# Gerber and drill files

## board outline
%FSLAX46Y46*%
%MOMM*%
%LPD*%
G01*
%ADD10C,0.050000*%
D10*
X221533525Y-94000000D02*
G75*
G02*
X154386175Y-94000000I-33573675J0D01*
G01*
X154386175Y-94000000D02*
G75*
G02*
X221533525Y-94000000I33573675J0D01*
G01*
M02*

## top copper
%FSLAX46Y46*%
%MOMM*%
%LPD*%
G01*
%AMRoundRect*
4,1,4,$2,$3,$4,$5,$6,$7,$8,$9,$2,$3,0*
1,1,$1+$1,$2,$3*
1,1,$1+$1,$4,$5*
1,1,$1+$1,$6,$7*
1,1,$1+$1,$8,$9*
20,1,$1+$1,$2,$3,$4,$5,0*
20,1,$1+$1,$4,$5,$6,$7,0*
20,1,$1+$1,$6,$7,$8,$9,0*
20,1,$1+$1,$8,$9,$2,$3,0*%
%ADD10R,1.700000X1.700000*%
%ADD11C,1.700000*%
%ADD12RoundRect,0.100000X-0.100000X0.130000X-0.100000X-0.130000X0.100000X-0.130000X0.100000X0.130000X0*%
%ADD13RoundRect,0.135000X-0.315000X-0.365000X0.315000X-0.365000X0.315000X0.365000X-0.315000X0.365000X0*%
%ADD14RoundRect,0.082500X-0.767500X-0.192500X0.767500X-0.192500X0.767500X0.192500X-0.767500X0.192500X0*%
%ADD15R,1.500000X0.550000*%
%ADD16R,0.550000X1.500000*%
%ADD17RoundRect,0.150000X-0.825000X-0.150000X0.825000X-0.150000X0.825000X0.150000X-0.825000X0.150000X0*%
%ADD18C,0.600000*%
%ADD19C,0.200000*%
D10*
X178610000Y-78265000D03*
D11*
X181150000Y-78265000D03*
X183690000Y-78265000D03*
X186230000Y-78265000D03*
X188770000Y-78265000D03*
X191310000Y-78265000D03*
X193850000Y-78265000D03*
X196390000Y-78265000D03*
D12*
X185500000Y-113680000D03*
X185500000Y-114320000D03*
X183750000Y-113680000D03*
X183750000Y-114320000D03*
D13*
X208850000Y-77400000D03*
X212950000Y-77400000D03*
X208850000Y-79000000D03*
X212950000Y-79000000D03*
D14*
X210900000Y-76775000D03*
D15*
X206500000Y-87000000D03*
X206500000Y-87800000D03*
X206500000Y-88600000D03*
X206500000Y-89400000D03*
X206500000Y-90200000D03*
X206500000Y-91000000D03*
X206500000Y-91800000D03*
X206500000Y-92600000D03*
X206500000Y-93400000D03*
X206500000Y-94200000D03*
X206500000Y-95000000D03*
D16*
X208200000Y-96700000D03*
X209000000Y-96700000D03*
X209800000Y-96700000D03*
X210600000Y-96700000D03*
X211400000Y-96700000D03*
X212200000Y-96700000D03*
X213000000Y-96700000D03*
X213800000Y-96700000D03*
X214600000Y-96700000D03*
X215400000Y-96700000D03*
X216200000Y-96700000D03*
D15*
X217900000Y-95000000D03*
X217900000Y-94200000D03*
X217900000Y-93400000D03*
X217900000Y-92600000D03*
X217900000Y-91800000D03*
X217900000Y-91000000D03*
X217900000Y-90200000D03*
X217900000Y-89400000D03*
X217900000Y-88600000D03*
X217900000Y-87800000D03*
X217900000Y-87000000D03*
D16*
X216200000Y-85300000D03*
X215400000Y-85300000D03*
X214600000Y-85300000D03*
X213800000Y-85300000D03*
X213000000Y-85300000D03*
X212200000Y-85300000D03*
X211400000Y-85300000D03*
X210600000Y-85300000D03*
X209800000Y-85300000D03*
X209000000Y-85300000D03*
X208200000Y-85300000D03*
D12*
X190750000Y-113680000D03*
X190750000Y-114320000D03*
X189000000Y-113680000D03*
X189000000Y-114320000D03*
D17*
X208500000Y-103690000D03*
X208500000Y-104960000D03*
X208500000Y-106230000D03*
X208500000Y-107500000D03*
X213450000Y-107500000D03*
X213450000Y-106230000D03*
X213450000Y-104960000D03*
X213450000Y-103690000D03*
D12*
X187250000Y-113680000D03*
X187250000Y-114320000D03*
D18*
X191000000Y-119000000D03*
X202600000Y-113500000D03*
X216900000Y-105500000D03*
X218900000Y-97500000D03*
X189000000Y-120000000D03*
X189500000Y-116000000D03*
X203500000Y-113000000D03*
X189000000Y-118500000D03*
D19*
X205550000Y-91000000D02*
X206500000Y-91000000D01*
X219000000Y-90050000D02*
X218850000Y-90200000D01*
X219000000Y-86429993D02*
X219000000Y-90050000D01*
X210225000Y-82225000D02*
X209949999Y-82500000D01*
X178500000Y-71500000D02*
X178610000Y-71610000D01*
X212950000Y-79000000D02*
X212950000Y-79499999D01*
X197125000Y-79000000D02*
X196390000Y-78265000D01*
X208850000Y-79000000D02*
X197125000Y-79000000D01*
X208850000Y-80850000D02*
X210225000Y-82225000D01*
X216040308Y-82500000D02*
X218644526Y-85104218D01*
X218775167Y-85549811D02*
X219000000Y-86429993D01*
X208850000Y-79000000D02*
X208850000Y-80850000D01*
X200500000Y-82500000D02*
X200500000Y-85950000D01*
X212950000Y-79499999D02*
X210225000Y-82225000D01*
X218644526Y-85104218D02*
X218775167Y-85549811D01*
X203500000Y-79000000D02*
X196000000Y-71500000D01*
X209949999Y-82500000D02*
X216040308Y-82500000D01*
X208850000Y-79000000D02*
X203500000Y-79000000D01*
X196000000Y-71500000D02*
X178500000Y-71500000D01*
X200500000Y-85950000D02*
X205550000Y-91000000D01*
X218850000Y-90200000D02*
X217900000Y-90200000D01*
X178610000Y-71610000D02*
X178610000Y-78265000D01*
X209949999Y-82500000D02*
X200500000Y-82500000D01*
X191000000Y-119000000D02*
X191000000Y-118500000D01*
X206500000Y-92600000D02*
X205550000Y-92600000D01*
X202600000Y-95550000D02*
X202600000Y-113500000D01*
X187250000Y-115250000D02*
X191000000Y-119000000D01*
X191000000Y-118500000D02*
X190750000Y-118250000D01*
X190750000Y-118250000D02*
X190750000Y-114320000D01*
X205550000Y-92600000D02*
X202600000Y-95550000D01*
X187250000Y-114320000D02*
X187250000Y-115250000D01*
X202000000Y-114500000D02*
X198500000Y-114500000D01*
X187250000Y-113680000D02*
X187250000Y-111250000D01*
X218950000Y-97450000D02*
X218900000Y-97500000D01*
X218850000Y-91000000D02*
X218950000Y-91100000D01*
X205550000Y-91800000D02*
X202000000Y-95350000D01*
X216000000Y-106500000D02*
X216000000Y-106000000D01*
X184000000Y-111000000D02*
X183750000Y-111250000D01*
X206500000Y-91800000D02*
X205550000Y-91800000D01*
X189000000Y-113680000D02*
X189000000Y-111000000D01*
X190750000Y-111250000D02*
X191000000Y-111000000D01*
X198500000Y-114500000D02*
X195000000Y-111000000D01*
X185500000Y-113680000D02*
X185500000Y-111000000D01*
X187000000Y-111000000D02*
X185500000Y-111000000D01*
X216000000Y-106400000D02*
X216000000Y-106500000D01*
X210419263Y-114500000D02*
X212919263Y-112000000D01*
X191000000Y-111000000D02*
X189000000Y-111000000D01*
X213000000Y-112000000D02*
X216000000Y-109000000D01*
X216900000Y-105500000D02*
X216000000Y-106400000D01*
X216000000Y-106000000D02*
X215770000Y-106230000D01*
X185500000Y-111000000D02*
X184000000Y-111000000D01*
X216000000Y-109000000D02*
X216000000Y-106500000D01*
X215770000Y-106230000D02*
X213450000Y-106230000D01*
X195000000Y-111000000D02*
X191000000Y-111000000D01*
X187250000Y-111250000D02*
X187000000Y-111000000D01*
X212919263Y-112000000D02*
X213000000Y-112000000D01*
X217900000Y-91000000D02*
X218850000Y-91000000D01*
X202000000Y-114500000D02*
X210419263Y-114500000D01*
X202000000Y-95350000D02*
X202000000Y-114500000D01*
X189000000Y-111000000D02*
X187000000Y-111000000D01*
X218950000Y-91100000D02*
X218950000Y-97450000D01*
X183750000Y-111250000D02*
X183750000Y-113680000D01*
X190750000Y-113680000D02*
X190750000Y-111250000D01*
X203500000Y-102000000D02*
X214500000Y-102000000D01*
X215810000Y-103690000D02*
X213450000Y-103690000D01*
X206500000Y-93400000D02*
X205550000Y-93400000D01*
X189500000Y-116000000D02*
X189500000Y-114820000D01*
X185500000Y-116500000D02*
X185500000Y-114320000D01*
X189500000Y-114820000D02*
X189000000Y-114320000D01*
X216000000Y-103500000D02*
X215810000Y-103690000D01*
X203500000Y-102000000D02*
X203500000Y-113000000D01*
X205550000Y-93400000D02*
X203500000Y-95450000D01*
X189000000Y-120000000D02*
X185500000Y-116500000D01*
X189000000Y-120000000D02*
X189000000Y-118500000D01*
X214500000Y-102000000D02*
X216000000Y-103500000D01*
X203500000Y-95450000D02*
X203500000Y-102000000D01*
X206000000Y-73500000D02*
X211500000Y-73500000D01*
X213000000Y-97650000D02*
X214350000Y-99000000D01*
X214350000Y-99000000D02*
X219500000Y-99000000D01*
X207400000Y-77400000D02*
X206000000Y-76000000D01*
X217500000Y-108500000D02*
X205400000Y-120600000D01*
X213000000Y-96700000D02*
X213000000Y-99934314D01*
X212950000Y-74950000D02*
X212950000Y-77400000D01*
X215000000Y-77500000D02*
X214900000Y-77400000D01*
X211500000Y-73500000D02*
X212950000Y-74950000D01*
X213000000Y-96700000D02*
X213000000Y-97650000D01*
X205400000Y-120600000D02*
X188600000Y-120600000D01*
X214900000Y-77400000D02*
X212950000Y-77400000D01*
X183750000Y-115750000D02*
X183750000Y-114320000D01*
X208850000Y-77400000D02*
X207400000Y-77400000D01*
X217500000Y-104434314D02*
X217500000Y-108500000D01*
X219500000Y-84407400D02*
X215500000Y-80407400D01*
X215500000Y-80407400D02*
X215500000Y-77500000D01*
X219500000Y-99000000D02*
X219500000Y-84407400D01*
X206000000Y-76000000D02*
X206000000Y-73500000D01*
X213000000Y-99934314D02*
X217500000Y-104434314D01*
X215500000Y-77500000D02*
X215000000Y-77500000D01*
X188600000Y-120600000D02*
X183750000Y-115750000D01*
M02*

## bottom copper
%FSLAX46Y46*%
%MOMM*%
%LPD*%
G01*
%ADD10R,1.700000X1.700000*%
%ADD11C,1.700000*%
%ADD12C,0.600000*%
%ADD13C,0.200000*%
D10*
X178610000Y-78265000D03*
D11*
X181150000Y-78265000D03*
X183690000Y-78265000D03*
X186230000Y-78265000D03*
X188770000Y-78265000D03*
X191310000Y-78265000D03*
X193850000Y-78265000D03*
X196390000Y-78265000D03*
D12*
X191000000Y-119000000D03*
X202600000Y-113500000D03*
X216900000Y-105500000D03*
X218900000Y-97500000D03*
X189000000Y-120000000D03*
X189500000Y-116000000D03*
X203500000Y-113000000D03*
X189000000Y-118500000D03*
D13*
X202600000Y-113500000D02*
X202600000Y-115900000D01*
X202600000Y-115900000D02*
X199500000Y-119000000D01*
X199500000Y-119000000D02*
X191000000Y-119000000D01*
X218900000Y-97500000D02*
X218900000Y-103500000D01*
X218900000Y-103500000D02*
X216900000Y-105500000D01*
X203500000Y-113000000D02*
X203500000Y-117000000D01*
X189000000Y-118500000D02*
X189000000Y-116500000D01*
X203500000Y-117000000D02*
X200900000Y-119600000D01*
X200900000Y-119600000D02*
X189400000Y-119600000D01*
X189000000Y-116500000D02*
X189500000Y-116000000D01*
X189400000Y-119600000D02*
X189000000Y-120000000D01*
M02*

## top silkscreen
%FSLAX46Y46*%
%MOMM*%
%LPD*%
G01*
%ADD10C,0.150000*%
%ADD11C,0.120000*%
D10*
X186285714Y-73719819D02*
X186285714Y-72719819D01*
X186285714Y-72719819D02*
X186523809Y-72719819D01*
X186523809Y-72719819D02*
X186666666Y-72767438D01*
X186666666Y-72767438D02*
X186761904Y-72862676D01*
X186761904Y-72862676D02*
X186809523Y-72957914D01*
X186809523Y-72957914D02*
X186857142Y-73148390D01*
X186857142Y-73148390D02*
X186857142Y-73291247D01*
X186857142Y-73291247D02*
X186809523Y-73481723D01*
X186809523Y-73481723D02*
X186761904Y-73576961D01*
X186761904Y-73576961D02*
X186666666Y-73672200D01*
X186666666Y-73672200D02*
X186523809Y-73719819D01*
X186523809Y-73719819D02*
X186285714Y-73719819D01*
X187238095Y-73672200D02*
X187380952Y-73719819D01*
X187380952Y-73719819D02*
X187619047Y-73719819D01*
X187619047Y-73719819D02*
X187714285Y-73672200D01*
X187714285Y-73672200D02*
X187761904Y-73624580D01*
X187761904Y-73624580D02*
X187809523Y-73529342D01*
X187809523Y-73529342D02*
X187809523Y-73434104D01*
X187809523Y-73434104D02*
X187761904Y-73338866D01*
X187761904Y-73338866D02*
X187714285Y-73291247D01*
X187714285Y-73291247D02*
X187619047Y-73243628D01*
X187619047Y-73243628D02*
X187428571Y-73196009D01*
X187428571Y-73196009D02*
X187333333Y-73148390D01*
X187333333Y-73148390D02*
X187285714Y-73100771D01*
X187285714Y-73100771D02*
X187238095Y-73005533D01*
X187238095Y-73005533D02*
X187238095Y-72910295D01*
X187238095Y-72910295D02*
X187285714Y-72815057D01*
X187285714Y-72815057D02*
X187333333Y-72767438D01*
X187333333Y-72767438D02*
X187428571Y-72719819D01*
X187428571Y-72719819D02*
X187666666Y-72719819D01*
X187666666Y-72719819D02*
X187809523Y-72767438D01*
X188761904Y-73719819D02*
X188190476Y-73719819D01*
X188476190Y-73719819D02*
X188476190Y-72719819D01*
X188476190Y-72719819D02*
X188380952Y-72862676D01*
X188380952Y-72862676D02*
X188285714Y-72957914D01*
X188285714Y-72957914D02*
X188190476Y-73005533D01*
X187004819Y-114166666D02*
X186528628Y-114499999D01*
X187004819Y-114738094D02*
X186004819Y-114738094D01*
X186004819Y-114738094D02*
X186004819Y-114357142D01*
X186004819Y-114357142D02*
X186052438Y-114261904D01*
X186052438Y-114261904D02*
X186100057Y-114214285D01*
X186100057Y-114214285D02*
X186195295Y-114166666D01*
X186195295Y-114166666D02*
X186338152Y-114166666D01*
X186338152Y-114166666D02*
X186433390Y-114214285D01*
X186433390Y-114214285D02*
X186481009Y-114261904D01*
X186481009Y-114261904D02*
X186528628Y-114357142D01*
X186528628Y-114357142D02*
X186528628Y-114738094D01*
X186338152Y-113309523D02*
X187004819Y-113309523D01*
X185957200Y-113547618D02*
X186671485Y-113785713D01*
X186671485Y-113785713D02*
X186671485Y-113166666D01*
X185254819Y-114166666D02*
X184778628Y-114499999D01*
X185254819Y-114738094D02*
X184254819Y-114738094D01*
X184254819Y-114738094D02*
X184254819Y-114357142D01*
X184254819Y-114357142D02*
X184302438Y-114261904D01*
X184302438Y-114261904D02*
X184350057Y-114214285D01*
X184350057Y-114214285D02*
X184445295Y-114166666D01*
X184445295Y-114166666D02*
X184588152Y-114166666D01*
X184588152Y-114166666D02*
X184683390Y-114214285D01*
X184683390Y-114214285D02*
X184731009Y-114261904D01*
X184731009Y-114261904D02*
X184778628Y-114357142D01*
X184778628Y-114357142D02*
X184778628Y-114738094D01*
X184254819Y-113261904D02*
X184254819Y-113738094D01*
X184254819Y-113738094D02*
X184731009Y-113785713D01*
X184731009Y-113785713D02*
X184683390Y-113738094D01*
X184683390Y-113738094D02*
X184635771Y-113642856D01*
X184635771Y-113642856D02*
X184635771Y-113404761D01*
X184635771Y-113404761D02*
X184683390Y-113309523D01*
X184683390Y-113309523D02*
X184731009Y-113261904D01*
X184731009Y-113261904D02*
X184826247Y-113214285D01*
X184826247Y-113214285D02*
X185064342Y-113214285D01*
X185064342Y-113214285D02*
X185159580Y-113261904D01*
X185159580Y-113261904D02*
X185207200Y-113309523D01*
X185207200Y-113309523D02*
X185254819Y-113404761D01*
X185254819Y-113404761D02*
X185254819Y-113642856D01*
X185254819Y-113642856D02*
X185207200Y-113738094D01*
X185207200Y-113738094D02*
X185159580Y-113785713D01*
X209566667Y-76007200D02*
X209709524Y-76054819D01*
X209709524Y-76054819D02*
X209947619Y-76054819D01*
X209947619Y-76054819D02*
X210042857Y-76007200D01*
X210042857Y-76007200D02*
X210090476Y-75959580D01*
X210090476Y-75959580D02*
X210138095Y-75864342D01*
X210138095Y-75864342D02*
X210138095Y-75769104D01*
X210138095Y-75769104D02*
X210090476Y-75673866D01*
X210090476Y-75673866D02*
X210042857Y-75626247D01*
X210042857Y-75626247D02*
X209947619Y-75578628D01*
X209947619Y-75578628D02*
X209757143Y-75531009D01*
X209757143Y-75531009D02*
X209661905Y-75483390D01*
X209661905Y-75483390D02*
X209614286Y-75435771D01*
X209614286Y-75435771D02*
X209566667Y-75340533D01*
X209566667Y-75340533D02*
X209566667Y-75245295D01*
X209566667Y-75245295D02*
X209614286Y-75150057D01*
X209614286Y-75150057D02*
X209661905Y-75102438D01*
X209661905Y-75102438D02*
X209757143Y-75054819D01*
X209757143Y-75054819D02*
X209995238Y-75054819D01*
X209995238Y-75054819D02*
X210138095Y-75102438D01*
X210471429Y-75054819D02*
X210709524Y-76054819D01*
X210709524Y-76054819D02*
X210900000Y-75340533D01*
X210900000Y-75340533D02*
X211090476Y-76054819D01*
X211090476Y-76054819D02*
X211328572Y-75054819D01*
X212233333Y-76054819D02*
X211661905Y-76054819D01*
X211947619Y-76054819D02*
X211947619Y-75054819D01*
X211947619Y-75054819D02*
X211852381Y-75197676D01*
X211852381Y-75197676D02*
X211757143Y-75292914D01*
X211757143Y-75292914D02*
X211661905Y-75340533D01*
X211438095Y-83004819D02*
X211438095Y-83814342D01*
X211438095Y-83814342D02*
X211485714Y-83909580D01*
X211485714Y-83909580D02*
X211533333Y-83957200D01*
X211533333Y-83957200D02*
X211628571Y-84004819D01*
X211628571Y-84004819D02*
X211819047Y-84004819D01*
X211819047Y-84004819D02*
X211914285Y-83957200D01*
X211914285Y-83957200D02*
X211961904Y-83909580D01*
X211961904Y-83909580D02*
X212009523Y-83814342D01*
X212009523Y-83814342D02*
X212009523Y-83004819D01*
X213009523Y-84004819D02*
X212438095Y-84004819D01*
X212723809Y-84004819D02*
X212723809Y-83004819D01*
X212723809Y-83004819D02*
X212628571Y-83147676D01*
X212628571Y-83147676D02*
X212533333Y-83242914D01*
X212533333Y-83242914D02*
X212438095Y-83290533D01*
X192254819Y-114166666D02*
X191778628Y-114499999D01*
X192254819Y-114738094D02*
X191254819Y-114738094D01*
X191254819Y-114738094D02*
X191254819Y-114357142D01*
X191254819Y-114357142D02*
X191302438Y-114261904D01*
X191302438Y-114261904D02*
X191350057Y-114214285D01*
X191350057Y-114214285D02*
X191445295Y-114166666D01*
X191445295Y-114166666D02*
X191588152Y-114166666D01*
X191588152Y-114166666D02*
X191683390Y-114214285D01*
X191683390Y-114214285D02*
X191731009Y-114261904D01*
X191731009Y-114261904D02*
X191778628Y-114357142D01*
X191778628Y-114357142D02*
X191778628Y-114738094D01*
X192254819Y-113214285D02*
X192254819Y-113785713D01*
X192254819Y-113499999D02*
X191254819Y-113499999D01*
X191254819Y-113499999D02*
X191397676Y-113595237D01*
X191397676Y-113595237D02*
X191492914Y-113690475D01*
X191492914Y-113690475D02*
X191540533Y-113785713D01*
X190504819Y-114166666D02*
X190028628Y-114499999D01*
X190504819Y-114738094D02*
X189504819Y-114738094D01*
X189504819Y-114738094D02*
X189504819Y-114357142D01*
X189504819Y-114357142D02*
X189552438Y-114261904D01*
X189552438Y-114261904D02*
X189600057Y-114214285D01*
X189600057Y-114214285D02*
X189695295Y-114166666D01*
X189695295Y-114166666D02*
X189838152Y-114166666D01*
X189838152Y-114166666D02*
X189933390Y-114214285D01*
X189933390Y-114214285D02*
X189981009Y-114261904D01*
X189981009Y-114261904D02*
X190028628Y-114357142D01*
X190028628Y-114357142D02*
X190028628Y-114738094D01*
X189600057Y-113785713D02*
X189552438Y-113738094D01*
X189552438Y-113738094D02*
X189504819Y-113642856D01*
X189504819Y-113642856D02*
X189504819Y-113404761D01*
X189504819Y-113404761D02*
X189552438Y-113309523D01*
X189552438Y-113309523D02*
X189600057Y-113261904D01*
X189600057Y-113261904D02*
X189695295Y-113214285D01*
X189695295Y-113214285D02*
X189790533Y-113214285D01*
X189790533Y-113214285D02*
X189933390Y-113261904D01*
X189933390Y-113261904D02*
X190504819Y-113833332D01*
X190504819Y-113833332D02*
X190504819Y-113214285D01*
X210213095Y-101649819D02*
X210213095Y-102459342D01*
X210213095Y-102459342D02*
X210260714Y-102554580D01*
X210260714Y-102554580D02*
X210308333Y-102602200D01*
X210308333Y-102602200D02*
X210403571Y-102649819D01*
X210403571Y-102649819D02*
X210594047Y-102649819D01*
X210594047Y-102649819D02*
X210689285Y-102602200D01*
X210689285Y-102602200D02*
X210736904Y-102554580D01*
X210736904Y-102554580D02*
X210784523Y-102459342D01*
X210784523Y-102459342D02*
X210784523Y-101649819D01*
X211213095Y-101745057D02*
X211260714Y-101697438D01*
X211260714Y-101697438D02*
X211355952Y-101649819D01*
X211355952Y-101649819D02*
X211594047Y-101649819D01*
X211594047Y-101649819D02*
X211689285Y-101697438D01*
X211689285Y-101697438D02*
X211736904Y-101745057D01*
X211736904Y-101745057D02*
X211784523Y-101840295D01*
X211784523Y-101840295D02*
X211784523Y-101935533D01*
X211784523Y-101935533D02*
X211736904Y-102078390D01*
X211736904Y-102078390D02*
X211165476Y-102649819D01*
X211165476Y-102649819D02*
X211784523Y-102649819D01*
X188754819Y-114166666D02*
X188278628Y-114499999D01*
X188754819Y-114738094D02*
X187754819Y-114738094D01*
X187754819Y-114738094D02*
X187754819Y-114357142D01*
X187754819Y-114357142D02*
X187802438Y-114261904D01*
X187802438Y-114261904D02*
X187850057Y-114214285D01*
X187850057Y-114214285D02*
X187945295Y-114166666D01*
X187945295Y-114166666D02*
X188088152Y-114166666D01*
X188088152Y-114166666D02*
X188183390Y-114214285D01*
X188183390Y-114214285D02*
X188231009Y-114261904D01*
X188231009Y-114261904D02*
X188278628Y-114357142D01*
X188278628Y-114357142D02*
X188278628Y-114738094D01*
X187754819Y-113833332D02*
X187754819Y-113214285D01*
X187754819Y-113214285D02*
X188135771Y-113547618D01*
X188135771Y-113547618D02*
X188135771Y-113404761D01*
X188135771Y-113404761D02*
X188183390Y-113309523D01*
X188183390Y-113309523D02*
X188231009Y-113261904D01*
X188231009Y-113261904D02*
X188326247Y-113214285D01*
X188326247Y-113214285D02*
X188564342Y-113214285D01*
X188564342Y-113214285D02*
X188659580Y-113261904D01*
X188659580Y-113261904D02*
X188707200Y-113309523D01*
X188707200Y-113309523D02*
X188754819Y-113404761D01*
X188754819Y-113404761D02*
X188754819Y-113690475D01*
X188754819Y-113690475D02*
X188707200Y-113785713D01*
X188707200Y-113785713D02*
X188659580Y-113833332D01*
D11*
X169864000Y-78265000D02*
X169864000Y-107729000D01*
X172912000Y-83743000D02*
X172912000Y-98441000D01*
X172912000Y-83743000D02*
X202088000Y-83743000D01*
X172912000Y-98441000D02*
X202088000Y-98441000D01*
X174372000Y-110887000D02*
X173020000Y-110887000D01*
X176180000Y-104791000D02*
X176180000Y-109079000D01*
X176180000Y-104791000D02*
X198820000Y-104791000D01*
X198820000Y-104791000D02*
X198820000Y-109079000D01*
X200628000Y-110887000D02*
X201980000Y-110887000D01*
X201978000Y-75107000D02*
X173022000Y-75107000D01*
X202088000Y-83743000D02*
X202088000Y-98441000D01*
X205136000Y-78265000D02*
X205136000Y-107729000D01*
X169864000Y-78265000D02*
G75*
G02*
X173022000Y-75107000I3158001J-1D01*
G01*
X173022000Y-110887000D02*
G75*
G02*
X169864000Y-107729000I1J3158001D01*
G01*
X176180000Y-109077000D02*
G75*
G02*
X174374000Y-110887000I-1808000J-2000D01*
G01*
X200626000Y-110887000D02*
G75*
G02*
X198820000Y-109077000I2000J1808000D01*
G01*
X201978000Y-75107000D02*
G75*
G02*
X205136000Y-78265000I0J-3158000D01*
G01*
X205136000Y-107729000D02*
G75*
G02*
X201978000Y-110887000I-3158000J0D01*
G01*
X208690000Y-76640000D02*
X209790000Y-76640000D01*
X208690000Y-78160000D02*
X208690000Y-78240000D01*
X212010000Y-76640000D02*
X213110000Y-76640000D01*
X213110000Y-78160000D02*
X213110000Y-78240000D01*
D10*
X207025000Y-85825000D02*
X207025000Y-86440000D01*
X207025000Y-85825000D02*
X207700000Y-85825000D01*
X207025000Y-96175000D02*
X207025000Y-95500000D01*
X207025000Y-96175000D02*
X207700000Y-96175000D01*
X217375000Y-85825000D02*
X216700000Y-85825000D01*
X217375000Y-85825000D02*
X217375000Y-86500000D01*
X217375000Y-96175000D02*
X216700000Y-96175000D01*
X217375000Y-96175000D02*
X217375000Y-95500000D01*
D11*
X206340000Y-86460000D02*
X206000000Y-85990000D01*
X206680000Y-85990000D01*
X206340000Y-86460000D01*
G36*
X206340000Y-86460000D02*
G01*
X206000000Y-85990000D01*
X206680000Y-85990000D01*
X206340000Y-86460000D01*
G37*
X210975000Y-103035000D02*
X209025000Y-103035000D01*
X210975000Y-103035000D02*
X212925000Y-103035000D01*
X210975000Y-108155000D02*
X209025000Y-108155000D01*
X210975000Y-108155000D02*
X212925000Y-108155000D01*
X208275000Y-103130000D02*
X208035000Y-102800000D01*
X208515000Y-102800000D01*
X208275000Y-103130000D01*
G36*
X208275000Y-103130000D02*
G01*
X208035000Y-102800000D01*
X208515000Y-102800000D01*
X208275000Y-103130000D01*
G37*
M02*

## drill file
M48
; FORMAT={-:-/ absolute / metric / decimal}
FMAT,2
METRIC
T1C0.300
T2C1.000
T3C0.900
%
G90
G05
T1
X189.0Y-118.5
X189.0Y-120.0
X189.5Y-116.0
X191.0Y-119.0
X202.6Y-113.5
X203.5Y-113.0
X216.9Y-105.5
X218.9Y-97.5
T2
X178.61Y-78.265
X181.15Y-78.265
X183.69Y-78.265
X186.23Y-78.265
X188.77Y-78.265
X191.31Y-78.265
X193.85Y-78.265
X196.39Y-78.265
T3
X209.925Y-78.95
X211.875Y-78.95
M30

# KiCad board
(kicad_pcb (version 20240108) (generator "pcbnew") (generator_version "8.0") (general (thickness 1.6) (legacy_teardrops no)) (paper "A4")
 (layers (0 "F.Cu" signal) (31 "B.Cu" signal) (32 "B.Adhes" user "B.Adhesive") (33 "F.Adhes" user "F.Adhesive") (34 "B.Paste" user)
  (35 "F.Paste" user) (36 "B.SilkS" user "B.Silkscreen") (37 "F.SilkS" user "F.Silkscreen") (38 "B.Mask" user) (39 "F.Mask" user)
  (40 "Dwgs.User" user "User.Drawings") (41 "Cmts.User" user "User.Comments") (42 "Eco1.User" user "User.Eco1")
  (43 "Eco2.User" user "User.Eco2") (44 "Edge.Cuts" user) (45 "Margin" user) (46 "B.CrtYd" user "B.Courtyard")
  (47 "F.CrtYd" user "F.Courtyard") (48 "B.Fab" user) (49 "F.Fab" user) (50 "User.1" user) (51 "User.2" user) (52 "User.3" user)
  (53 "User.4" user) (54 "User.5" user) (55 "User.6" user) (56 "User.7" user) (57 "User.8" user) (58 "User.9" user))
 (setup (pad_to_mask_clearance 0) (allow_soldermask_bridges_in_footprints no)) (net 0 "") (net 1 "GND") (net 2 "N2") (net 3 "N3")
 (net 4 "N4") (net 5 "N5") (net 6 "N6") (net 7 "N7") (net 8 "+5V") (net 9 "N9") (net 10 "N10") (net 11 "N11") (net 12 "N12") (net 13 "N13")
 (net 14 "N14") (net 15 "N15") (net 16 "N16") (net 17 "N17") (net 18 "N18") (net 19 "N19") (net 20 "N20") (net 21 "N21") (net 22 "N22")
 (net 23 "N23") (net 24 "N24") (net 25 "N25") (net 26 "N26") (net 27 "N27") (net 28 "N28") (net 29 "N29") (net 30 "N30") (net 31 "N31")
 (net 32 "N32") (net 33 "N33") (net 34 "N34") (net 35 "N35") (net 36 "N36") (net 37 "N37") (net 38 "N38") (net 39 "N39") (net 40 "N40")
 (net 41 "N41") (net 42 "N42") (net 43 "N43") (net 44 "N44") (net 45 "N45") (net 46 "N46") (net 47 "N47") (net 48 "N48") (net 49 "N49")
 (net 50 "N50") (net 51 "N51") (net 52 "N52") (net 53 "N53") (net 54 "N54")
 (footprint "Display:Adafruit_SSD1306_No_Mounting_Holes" (layer "F.Cu") (at 178.61 78.265)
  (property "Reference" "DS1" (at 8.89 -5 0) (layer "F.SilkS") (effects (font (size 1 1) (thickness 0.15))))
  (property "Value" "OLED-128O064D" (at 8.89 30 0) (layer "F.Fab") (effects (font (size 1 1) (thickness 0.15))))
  (fp_line (start -8.746 0) (end -8.746 29.464) (stroke (width 0.12) (type solid)) (layer "F.SilkS"))
  (fp_line (start -5.698 5.478) (end -5.698 20.176) (stroke (width 0.12) (type solid)) (layer "F.SilkS"))
  (fp_line (start -5.698 5.478) (end 23.478 5.478) (stroke (width 0.12) (type solid)) (layer "F.SilkS"))
  (fp_line (start -5.698 20.176) (end 23.478 20.176) (stroke (width 0.12) (type solid)) (layer "F.SilkS"))
  (fp_line (start -4.238 32.622) (end -5.59 32.622) (stroke (width 0.12) (type solid)) (layer "F.SilkS"))
  (fp_line (start -2.43 26.526) (end -2.43 30.814) (stroke (width 0.12) (type solid)) (layer "F.SilkS"))
  (fp_line (start -2.43 26.526) (end 20.21 26.526) (stroke (width 0.12) (type solid)) (layer "F.SilkS"))
  (fp_line (start 20.21 26.526) (end 20.21 30.814) (stroke (width 0.12) (type solid)) (layer "F.SilkS"))
  (fp_line (start 22.018 32.622) (end 23.37 32.622) (stroke (width 0.12) (type solid)) (layer "F.SilkS"))
  (fp_line (start 23.368 -3.158) (end -5.588 -3.158) (stroke (width 0.12) (type solid)) (layer "F.SilkS"))
  (fp_line (start 23.478 5.478) (end 23.478 20.176) (stroke (width 0.12) (type solid)) (layer "F.SilkS"))
  (fp_line (start 26.526 0) (end 26.526 29.464) (stroke (width 0.12) (type solid)) (layer "F.SilkS"))
  (fp_arc (start -8.746 0) (mid -7.821043 -2.233043) (end -5.588 -3.158) (stroke (width 0.12) (type solid)) (layer "F.SilkS"))
  (fp_arc (start -5.588 32.622) (mid -7.821043 31.697043) (end -8.746 29.464) (stroke (width 0.12) (type solid)) (layer "F.SilkS"))
  (fp_arc (start -2.43 30.812) (mid -2.958137 32.091035) (end -4.236 32.622) (stroke (width 0.12) (type solid)) (layer "F.SilkS"))
  (fp_arc (start 22.016 32.622) (mid 20.738137 32.091035) (end 20.21 30.812) (stroke (width 0.12) (type solid)) (layer "F.SilkS"))
  (fp_arc (start 23.368 -3.158) (mid 25.601043 -2.233043) (end 26.526 0) (stroke (width 0.12) (type solid)) (layer "F.SilkS"))
  (fp_arc (start 26.526 29.464) (mid 25.601043 31.697043) (end 23.368 32.622) (stroke (width 0.12) (type solid)) (layer "F.SilkS"))
  (pad "1" thru_hole rect (at 0 0) (size 1.7 1.7) (drill 1) (layers "*.Cu" "*.Mask") (remove_unused_layers no) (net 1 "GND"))
  (pad "2" thru_hole circle (at 2.54 0) (size 1.7 1.7) (drill 1) (layers "*.Cu" "*.Mask") (remove_unused_layers no) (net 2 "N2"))
  (pad "3" thru_hole circle (at 5.08 0) (size 1.7 1.7) (drill 1) (layers "*.Cu" "*.Mask") (remove_unused_layers no) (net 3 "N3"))
  (pad "4" thru_hole circle (at 7.62 0) (size 1.7 1.7) (drill 1) (layers "*.Cu" "*.Mask") (remove_unused_layers no) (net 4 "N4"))
  (pad "5" thru_hole circle (at 10.16 0) (size 1.7 1.7) (drill 1) (layers "*.Cu" "*.Mask") (remove_unused_layers no) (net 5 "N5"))
  (pad "6" thru_hole circle (at 12.7 0) (size 1.7 1.7) (drill 1) (layers "*.Cu" "*.Mask") (remove_unused_layers no) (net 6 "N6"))
  (pad "7" thru_hole circle (at 15.24 0) (size 1.7 1.7) (drill 1) (layers "*.Cu" "*.Mask") (remove_unused_layers no) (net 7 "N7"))
  (pad "8" thru_hole circle (at 17.78 0) (size 1.7 1.7) (drill 1) (layers "*.Cu" "*.Mask") (remove_unused_layers no) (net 1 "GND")))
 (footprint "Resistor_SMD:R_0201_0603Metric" (layer "F.Cu") (at 185.5 114 -90)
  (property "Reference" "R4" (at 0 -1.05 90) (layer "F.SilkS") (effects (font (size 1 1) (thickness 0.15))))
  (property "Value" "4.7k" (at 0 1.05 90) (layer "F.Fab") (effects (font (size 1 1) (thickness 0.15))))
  (pad "" smd roundrect (at -0.345 0 270) (size 0.318 0.36) (layers "F.Paste") (roundrect_rratio 0.25))
  (pad "" smd roundrect (at 0.345 0 270) (size 0.318 0.36) (layers "F.Paste") (roundrect_rratio 0.25))
  (pad "1" smd roundrect (at -0.32 0 270) (size 0.46 0.4) (layers "F.Cu" "F.Mask") (roundrect_rratio 0.25) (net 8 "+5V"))
  (pad "2" smd roundrect (at 0.32 0 270) (size 0.46 0.4) (layers "F.Cu" "F.Mask") (roundrect_rratio 0.25) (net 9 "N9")))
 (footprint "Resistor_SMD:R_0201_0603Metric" (layer "F.Cu") (at 183.75 114 -90)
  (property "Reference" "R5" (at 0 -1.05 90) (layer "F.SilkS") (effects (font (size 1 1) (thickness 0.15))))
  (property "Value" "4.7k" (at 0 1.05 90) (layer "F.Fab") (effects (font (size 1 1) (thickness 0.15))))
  (pad "" smd roundrect (at -0.345 0 270) (size 0.318 0.36) (layers "F.Paste") (roundrect_rratio 0.25))
  (pad "" smd roundrect (at 0.345 0 270) (size 0.318 0.36) (layers "F.Paste") (roundrect_rratio 0.25))
  (pad "1" smd roundrect (at -0.32 0 270) (size 0.46 0.4) (layers "F.Cu" "F.Mask") (roundrect_rratio 0.25) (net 8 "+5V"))
  (pad "2" smd roundrect (at 0.32 0 270) (size 0.46 0.4) (layers "F.Cu" "F.Mask") (roundrect_rratio 0.25) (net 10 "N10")))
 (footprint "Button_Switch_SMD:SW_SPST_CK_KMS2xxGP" (layer "F.Cu") (at 210.9 78.2)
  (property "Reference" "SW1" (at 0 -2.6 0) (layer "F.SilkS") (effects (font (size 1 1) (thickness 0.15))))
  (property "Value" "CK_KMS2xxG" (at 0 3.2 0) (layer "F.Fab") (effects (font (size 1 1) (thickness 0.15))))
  (fp_line (start -2.21 -1.56) (end -1.11 -1.56) (stroke (width 0.12) (type solid)) (layer "F.SilkS"))
  (fp_line (start -2.21 -0.04) (end -2.21 0.04) (stroke (width 0.12) (type default)) (layer "F.SilkS"))
  (fp_line (start 1.11 -1.56) (end 2.21 -1.56) (stroke (width 0.12) (type solid)) (layer "F.SilkS"))
  (fp_line (start 2.21 -0.04) (end 2.21 0.04) (stroke (width 0.12) (type default)) (layer "F.SilkS"))
  (pad "" np_thru_hole circle (at -0.975 0.75) (size 0.9 0.9) (drill 0.9) (layers "F&B.Cu" "*.Mask"))
  (pad "" np_thru_hole circle (at 0.975 0.75) (size 0.9 0.9) (drill 0.9) (layers "F&B.Cu" "*.Mask"))
  (pad "1" smd roundrect (at -2.05 -0.8) (size 0.9 1) (layers "F.Cu" "F.Paste" "F.Mask") (roundrect_rratio 0.15) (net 10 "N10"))
  (pad "1" smd roundrect (at 2.05 -0.8) (size 0.9 1) (layers "F.Cu" "F.Paste" "F.Mask") (roundrect_rratio 0.15) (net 10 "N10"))
  (pad "2" smd roundrect (at -2.05 0.8) (size 0.9 1) (layers "F.Cu" "F.Paste" "F.Mask") (roundrect_rratio 0.15) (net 1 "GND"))
  (pad "2" smd roundrect (at 2.05 0.8) (size 0.9 1) (layers "F.Cu" "F.Paste" "F.Mask") (roundrect_rratio 0.15) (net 1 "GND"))
  (pad "SH" smd roundrect (at 0 -1.425) (size 1.7 0.55) (layers "F.Cu" "F.Paste" "F.Mask") (roundrect_rratio 0.15) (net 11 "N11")))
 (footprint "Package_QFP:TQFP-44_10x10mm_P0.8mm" (layer "F.Cu") (at 212.2 91)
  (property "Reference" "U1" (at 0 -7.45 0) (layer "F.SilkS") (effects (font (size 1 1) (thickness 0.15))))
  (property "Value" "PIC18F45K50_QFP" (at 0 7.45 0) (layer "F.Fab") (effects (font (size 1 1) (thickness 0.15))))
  (fp_line (start -5.175 -5.175) (end -5.175 -4.56) (stroke (width 0.15) (type solid)) (layer "F.SilkS"))
  (fp_line (start -5.175 -5.175) (end -4.5 -5.175) (stroke (width 0.15) (type solid)) (layer "F.SilkS"))
  (fp_line (start -5.175 5.175) (end -5.175 4.5) (stroke (width 0.15) (type solid)) (layer "F.SilkS"))
  (fp_line (start -5.175 5.175) (end -4.5 5.175) (stroke (width 0.15) (type solid)) (layer "F.SilkS"))
  (fp_line (start 5.175 -5.175) (end 4.5 -5.175) (stroke (width 0.15) (type solid)) (layer "F.SilkS"))
  (fp_line (start 5.175 -5.175) (end 5.175 -4.5) (stroke (width 0.15) (type solid)) (layer "F.SilkS"))
  (fp_line (start 5.175 5.175) (end 4.5 5.175) (stroke (width 0.15) (type solid)) (layer "F.SilkS"))
  (fp_line (start 5.175 5.175) (end 5.175 4.5) (stroke (width 0.15) (type solid)) (layer "F.SilkS"))
  (fp_poly
   (pts (xy -5.86 -4.54) (xy -6.2 -5.01) (xy -5.52 -5.01) (xy -5.86 -4.54)) (stroke (width 0.12) (type solid)) (fill solid)
   (layer "F.SilkS"))
  (pad "1" smd rect (at -5.7 -4) (size 1.5 0.55) (layers "F.Cu" "F.Paste" "F.Mask") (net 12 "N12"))
  (pad "2" smd rect (at -5.7 -3.2) (size 1.5 0.55) (layers "F.Cu" "F.Paste" "F.Mask") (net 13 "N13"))
  (pad "3" smd rect (at -5.7 -2.4) (size 1.5 0.55) (layers "F.Cu" "F.Paste" "F.Mask") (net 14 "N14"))
  (pad "4" smd rect (at -5.7 -1.6) (size 1.5 0.55) (layers "F.Cu" "F.Paste" "F.Mask") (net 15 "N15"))
  (pad "5" smd rect (at -5.7 -0.8) (size 1.5 0.55) (layers "F.Cu" "F.Paste" "F.Mask") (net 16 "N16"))
  (pad "6" smd rect (at -5.7 0) (size 1.5 0.55) (layers "F.Cu" "F.Paste" "F.Mask") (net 1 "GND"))
  (pad "7" smd rect (at -5.7 0.8) (size 1.5 0.55) (layers "F.Cu" "F.Paste" "F.Mask") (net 8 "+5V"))
  (pad "8" smd rect (at -5.7 1.6) (size 1.5 0.55) (layers "F.Cu" "F.Paste" "F.Mask") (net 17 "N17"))
  (pad "9" smd rect (at -5.7 2.4) (size 1.5 0.55) (layers "F.Cu" "F.Paste" "F.Mask") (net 9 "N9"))
  (pad "10" smd rect (at -5.7 3.2) (size 1.5 0.55) (layers "F.Cu" "F.Paste" "F.Mask") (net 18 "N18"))
  (pad "11" smd rect (at -5.7 4) (size 1.5 0.55) (layers "F.Cu" "F.Paste" "F.Mask") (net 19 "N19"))
  (pad "12" smd rect (at -4 5.7 90) (size 1.5 0.55) (layers "F.Cu" "F.Paste" "F.Mask") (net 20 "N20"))
  (pad "13" smd rect (at -3.2 5.7 90) (size 1.5 0.55) (layers "F.Cu" "F.Paste" "F.Mask") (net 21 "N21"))
  (pad "14" smd rect (at -2.4 5.7 90) (size 1.5 0.55) (layers "F.Cu" "F.Paste" "F.Mask") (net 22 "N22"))
  (pad "15" smd rect (at -1.6 5.7 90) (size 1.5 0.55) (layers "F.Cu" "F.Paste" "F.Mask") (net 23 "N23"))
  (pad "16" smd rect (at -0.8 5.7 90) (size 1.5 0.55) (layers "F.Cu" "F.Paste" "F.Mask") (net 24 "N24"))
  (pad "17" smd rect (at 0 5.7 90) (size 1.5 0.55) (layers "F.Cu" "F.Paste" "F.Mask") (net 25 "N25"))
  (pad "18" smd rect (at 0.8 5.7 90) (size 1.5 0.55) (layers "F.Cu" "F.Paste" "F.Mask") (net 10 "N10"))
  (pad "19" smd rect (at 1.6 5.7 90) (size 1.5 0.55) (layers "F.Cu" "F.Paste" "F.Mask") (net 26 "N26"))
  (pad "20" smd rect (at 2.4 5.7 90) (size 1.5 0.55) (layers "F.Cu" "F.Paste" "F.Mask") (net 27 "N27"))
  (pad "21" smd rect (at 3.2 5.7 90) (size 1.5 0.55) (layers "F.Cu" "F.Paste" "F.Mask") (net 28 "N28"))
  (pad "22" smd rect (at 4 5.7 90) (size 1.5 0.55) (layers "F.Cu" "F.Paste" "F.Mask") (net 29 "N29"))
  (pad "23" smd rect (at 5.7 4) (size 1.5 0.55) (layers "F.Cu" "F.Paste" "F.Mask") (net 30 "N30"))
  (pad "24" smd rect (at 5.7 3.2) (size 1.5 0.55) (layers "F.Cu" "F.Paste" "F.Mask") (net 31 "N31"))
  (pad "25" smd rect (at 5.7 2.4) (size 1.5 0.55) (layers "F.Cu" "F.Paste" "F.Mask") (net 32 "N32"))
  (pad "26" smd rect (at 5.7 1.6) (size 1.5 0.55) (layers "F.Cu" "F.Paste" "F.Mask") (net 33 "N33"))
  (pad "27" smd rect (at 5.7 0.8) (size 1.5 0.55) (layers "F.Cu" "F.Paste" "F.Mask") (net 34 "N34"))
  (pad "28" smd rect (at 5.7 0) (size 1.5 0.55) (layers "F.Cu" "F.Paste" "F.Mask") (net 8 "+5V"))
  (pad "29" smd rect (at 5.7 -0.8) (size 1.5 0.55) (layers "F.Cu" "F.Paste" "F.Mask") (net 1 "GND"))
  (pad "30" smd rect (at 5.7 -1.6) (size 1.5 0.55) (layers "F.Cu" "F.Paste" "F.Mask") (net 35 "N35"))
  (pad "31" smd rect (at 5.7 -2.4) (size 1.5 0.55) (layers "F.Cu" "F.Paste" "F.Mask") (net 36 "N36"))
  (pad "32" smd rect (at 5.7 -3.2) (size 1.5 0.55) (layers "F.Cu" "F.Paste" "F.Mask") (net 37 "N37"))
  (pad "33" smd rect (at 5.7 -4) (size 1.5 0.55) (layers "F.Cu" "F.Paste" "F.Mask") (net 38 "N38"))
  (pad "34" smd rect (at 4 -5.7 90) (size 1.5 0.55) (layers "F.Cu" "F.Paste" "F.Mask") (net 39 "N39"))
  (pad "35" smd rect (at 3.2 -5.7 90) (size 1.5 0.55) (layers "F.Cu" "F.Paste" "F.Mask") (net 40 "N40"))
  (pad "36" smd rect (at 2.4 -5.7 90) (size 1.5 0.55) (layers "F.Cu" "F.Paste" "F.Mask") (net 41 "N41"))
  (pad "37" smd rect (at 1.6 -5.7 90) (size 1.5 0.55) (layers "F.Cu" "F.Paste" "F.Mask") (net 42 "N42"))
  (pad "38" smd rect (at 0.8 -5.7 90) (size 1.5 0.55) (layers "F.Cu" "F.Paste" "F.Mask") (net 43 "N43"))
  (pad "39" smd rect (at 0 -5.7 90) (size 1.5 0.55) (layers "F.Cu" "F.Paste" "F.Mask") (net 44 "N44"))
  (pad "40" smd rect (at -0.8 -5.7 90) (size 1.5 0.55) (layers "F.Cu" "F.Paste" "F.Mask") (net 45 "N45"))
  (pad "41" smd rect (at -1.6 -5.7 90) (size 1.5 0.55) (layers "F.Cu" "F.Paste" "F.Mask") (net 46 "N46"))
  (pad "42" smd rect (at -2.4 -5.7 90) (size 1.5 0.55) (layers "F.Cu" "F.Paste" "F.Mask") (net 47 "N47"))
  (pad "43" smd rect (at -3.2 -5.7 90) (size 1.5 0.55) (layers "F.Cu" "F.Paste" "F.Mask") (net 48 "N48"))
  (pad "44" smd rect (at -4 -5.7 90) (size 1.5 0.55) (layers "F.Cu" "F.Paste" "F.Mask") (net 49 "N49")))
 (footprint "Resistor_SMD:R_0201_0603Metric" (layer "F.Cu") (at 190.75 114 -90)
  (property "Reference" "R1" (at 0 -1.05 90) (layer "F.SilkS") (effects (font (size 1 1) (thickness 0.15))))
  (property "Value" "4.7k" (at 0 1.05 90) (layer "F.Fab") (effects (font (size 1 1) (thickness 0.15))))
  (pad "" smd roundrect (at -0.345 0 270) (size 0.318 0.36) (layers "F.Paste") (roundrect_rratio 0.25))
  (pad "" smd roundrect (at 0.345 0 270) (size 0.318 0.36) (layers "F.Paste") (roundrect_rratio 0.25))
  (pad "1" smd roundrect (at -0.32 0 270) (size 0.46 0.4) (layers "F.Cu" "F.Mask") (roundrect_rratio 0.25) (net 8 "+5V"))
  (pad "2" smd roundrect (at 0.32 0 270) (size 0.46 0.4) (layers "F.Cu" "F.Mask") (roundrect_rratio 0.25) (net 17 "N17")))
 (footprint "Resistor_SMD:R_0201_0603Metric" (layer "F.Cu") (at 189 114 -90)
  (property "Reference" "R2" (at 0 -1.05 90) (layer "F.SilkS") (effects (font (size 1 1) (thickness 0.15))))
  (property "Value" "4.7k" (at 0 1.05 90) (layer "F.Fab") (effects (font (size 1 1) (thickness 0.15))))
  (pad "" smd roundrect (at -0.345 0 270) (size 0.318 0.36) (layers "F.Paste") (roundrect_rratio 0.25))
  (pad "" smd roundrect (at 0.345 0 270) (size 0.318 0.36) (layers "F.Paste") (roundrect_rratio 0.25))
  (pad "1" smd roundrect (at -0.32 0 270) (size 0.46 0.4) (layers "F.Cu" "F.Mask") (roundrect_rratio 0.25) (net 8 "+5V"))
  (pad "2" smd roundrect (at 0.32 0 270) (size 0.46 0.4) (layers "F.Cu" "F.Mask") (roundrect_rratio 0.25) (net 9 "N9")))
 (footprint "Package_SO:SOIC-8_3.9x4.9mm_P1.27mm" (layer "F.Cu") (at 210.975 105.595)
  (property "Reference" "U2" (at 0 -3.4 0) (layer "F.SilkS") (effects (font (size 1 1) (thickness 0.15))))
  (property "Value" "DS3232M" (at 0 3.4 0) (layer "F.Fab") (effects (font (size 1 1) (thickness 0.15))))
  (fp_line (start 0 -2.56) (end -1.95 -2.56) (stroke (width 0.12) (type solid)) (layer "F.SilkS"))
  (fp_line (start 0 -2.56) (end 1.95 -2.56) (stroke (width 0.12) (type solid)) (layer "F.SilkS"))
  (fp_line (start 0 2.56) (end -1.95 2.56) (stroke (width 0.12) (type solid)) (layer "F.SilkS"))
  (fp_line (start 0 2.56) (end 1.95 2.56) (stroke (width 0.12) (type solid)) (layer "F.SilkS"))
  (fp_poly
   (pts (xy -2.7 -2.465) (xy -2.94 -2.795) (xy -2.46 -2.795) (xy -2.7 -2.465)) (stroke (width 0.12) (type solid)) (fill solid)
   (layer "F.SilkS"))
  (pad "1" smd roundrect (at -2.475 -1.905) (size 1.95 0.6) (layers "F.Cu" "F.Paste" "F.Mask") (roundrect_rratio 0.25) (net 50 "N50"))
  (pad "2" smd roundrect (at -2.475 -0.635) (size 1.95 0.6) (layers "F.Cu" "F.Paste" "F.Mask") (roundrect_rratio 0.25) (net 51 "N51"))
  (pad "3" smd roundrect (at -2.475 0.635) (size 1.95 0.6) (layers "F.Cu" "F.Paste" "F.Mask") (roundrect_rratio 0.25) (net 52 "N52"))
  (pad "4" smd roundrect (at -2.475 1.905) (size 1.95 0.6) (layers "F.Cu" "F.Paste" "F.Mask") (roundrect_rratio 0.25) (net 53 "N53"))
  (pad "5" smd roundrect (at 2.475 1.905) (size 1.95 0.6) (layers "F.Cu" "F.Paste" "F.Mask") (roundrect_rratio 0.25) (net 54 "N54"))
  (pad "6" smd roundrect (at 2.475 0.635) (size 1.95 0.6) (layers "F.Cu" "F.Paste" "F.Mask") (roundrect_rratio 0.25) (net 8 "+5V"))
  (pad "7" smd roundrect (at 2.475 -0.635) (size 1.95 0.6) (layers "F.Cu" "F.Paste" "F.Mask") (roundrect_rratio 0.25) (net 17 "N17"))
  (pad "8" smd roundrect (at 2.475 -1.905) (size 1.95 0.6) (layers "F.Cu" "F.Paste" "F.Mask") (roundrect_rratio 0.25) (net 9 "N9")))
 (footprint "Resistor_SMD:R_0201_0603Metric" (layer "F.Cu") (at 187.25 114 -90)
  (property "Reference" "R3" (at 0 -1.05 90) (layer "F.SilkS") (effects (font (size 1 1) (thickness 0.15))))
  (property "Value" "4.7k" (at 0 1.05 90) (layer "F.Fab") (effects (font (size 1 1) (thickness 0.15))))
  (pad "" smd roundrect (at -0.345 0 270) (size 0.318 0.36) (layers "F.Paste") (roundrect_rratio 0.25))
  (pad "" smd roundrect (at 0.345 0 270) (size 0.318 0.36) (layers "F.Paste") (roundrect_rratio 0.25))
  (pad "1" smd roundrect (at -0.32 0 270) (size 0.46 0.4) (layers "F.Cu" "F.Mask") (roundrect_rratio 0.25) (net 8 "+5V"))
  (pad "2" smd roundrect (at 0.32 0 270) (size 0.46 0.4) (layers "F.Cu" "F.Mask") (roundrect_rratio 0.25) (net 17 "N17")))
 (gr_circle (center 187.95985 94) (end 221.5 95.5) (stroke (width 0.05) (type default)) (fill none) (layer "Edge.Cuts"))
 (segment (start 205.55 91) (end 206.5 91) (width 0.2) (layer "F.Cu") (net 1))
 (segment (start 219 90.05) (end 218.85 90.2) (width 0.2) (layer "F.Cu") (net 1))
 (segment (start 219 86.429993) (end 219 90.05) (width 0.2) (layer "F.Cu") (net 1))
 (segment (start 210.225 82.225) (end 209.949999 82.5) (width 0.2) (layer "F.Cu") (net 1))
 (segment (start 178.5 71.5) (end 178.61 71.61) (width 0.2) (layer "F.Cu") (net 1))
 (segment (start 212.95 79) (end 212.95 79.499999) (width 0.2) (layer "F.Cu") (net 1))
 (segment (start 197.125 79) (end 196.39 78.265) (width 0.2) (layer "F.Cu") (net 1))
 (segment (start 208.85 79) (end 197.125 79) (width 0.2) (layer "F.Cu") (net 1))
 (segment (start 208.85 80.85) (end 210.225 82.225) (width 0.2) (layer "F.Cu") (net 1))
 (segment (start 216.040308 82.5) (end 218.644526 85.104218) (width 0.2) (layer "F.Cu") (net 1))
 (segment (start 218.775167 85.549811) (end 219 86.429993) (width 0.2) (layer "F.Cu") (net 1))
 (segment (start 208.85 79) (end 208.85 80.85) (width 0.2) (layer "F.Cu") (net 1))
 (segment (start 200.5 82.5) (end 200.5 85.95) (width 0.2) (layer "F.Cu") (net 1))
 (segment (start 212.95 79.499999) (end 210.225 82.225) (width 0.2) (layer "F.Cu") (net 1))
 (segment (start 218.644526 85.104218) (end 218.775167 85.549811) (width 0.2) (layer "F.Cu") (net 1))
 (segment (start 203.5 79) (end 196 71.5) (width 0.2) (layer "F.Cu") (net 1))
 (segment (start 209.949999 82.5) (end 216.040308 82.5) (width 0.2) (layer "F.Cu") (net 1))
 (segment (start 208.85 79) (end 203.5 79) (width 0.2) (layer "F.Cu") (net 1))
 (segment (start 196 71.5) (end 178.5 71.5) (width 0.2) (layer "F.Cu") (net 1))
 (segment (start 200.5 85.95) (end 205.55 91) (width 0.2) (layer "F.Cu") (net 1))
 (segment (start 218.85 90.2) (end 217.9 90.2) (width 0.2) (layer "F.Cu") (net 1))
 (segment (start 178.61 71.61) (end 178.61 78.265) (width 0.2) (layer "F.Cu") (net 1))
 (segment (start 209.949999 82.5) (end 200.5 82.5) (width 0.2) (layer "F.Cu") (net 1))
 (segment (start 191 119) (end 191 118.5) (width 0.2) (layer "F.Cu") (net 17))
 (segment (start 206.5 92.6) (end 205.55 92.6) (width 0.2) (layer "F.Cu") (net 17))
 (segment (start 202.6 95.55) (end 202.6 113.5) (width 0.2) (layer "F.Cu") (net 17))
 (segment (start 187.25 115.25) (end 191 119) (width 0.2) (layer "F.Cu") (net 17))
 (segment (start 191 118.5) (end 190.75 118.25) (width 0.2) (layer "F.Cu") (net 17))
 (segment (start 190.75 118.25) (end 190.75 114.32) (width 0.2) (layer "F.Cu") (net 17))
 (segment (start 205.55 92.6) (end 202.6 95.55) (width 0.2) (layer "F.Cu") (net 17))
 (segment (start 187.25 114.32) (end 187.25 115.25) (width 0.2) (layer "F.Cu") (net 17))
 (via (at 191 119) (size 0.6) (drill 0.3) (layers "F.Cu" "B.Cu") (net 17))
 (via (at 202.6 113.5) (size 0.6) (drill 0.3) (layers "F.Cu" "B.Cu") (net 17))
 (segment (start 202.6 113.5) (end 202.6 115.9) (width 0.2) (layer "B.Cu") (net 17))
 (segment (start 202.6 115.9) (end 199.5 119) (width 0.2) (layer "B.Cu") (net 17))
 (segment (start 199.5 119) (end 191 119) (width 0.2) (layer "B.Cu") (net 17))
 (segment (start 202 114.5) (end 198.5 114.5) (width 0.2) (layer "F.Cu") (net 8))
 (segment (start 187.25 113.68) (end 187.25 111.25) (width 0.2) (layer "F.Cu") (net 8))
 (segment (start 218.95 97.45) (end 218.9 97.5) (width 0.2) (layer "F.Cu") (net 8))
 (segment (start 218.85 91) (end 218.95 91.1) (width 0.2) (layer "F.Cu") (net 8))
 (segment (start 205.55 91.8) (end 202 95.35) (width 0.2) (layer "F.Cu") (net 8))
 (segment (start 216 106.5) (end 216 106) (width 0.2) (layer "F.Cu") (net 8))
 (segment (start 184 111) (end 183.75 111.25) (width 0.2) (layer "F.Cu") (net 8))
 (segment (start 206.5 91.8) (end 205.55 91.8) (width 0.2) (layer "F.Cu") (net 8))
 (segment (start 189 113.68) (end 189 111) (width 0.2) (layer "F.Cu") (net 8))
 (segment (start 190.75 111.25) (end 191 111) (width 0.2) (layer "F.Cu") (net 8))
 (segment (start 198.5 114.5) (end 195 111) (width 0.2) (layer "F.Cu") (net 8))
 (segment (start 185.5 113.68) (end 185.5 111) (width 0.2) (layer "F.Cu") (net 8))
 (segment (start 187 111) (end 185.5 111) (width 0.2) (layer "F.Cu") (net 8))
 (segment (start 216 106.4) (end 216 106.5) (width 0.2) (layer "F.Cu") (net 8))
 (segment (start 210.419263 114.5) (end 212.919263 112) (width 0.2) (layer "F.Cu") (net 8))
 (segment (start 191 111) (end 189 111) (width 0.2) (layer "F.Cu") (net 8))
 (segment (start 213 112) (end 216 109) (width 0.2) (layer "F.Cu") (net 8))
 (segment (start 216.9 105.5) (end 216 106.4) (width 0.2) (layer "F.Cu") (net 8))
 (segment (start 216 106) (end 215.77 106.23) (width 0.2) (layer "F.Cu") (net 8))
 (segment (start 185.5 111) (end 184 111) (width 0.2) (layer "F.Cu") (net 8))
 (segment (start 216 109) (end 216 106.5) (width 0.2) (layer "F.Cu") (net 8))
 (segment (start 215.77 106.23) (end 213.45 106.23) (width 0.2) (layer "F.Cu") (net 8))
 (segment (start 195 111) (end 191 111) (width 0.2) (layer "F.Cu") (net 8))
 (segment (start 187.25 111.25) (end 187 111) (width 0.2) (layer "F.Cu") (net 8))
 (segment (start 212.919263 112) (end 213 112) (width 0.2) (layer "F.Cu") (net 8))
 (segment (start 217.9 91) (end 218.85 91) (width 0.2) (layer "F.Cu") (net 8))
 (segment (start 202 114.5) (end 210.419263 114.5) (width 0.2) (layer "F.Cu") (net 8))
 (segment (start 202 95.35) (end 202 114.5) (width 0.2) (layer "F.Cu") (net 8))
 (segment (start 189 111) (end 187 111) (width 0.2) (layer "F.Cu") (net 8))
 (segment (start 218.95 91.1) (end 218.95 97.45) (width 0.2) (layer "F.Cu") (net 8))
 (segment (start 183.75 111.25) (end 183.75 113.68) (width 0.2) (layer "F.Cu") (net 8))
 (segment (start 190.75 113.68) (end 190.75 111.25) (width 0.2) (layer "F.Cu") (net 8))
 (via (at 216.9 105.5) (size 0.6) (drill 0.3) (layers "F.Cu" "B.Cu") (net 8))
 (via (at 218.9 97.5) (size 0.6) (drill 0.3) (layers "F.Cu" "B.Cu") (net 8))
 (segment (start 218.9 97.5) (end 218.9 103.5) (width 0.2) (layer "B.Cu") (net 8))
 (segment (start 218.9 103.5) (end 216.9 105.5) (width 0.2) (layer "B.Cu") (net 8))
 (segment (start 203.5 102) (end 214.5 102) (width 0.2) (layer "F.Cu") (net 9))
 (segment (start 215.81 103.69) (end 213.45 103.69) (width 0.2) (layer "F.Cu") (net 9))
 (segment (start 206.5 93.4) (end 205.55 93.4) (width 0.2) (layer "F.Cu") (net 9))
 (segment (start 189.5 116) (end 189.5 114.82) (width 0.2) (layer "F.Cu") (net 9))
 (segment (start 185.5 116.5) (end 185.5 114.32) (width 0.2) (layer "F.Cu") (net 9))
 (segment (start 189.5 114.82) (end 189 114.32) (width 0.2) (layer "F.Cu") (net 9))
 (segment (start 216 103.5) (end 215.81 103.69) (width 0.2) (layer "F.Cu") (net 9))
 (segment (start 203.5 102) (end 203.5 113) (width 0.2) (layer "F.Cu") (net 9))
 (segment (start 205.55 93.4) (end 203.5 95.45) (width 0.2) (layer "F.Cu") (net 9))
 (segment (start 189 120) (end 185.5 116.5) (width 0.2) (layer "F.Cu") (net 9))
 (segment (start 189 120) (end 189 118.5) (width 0.2) (layer "F.Cu") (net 9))
 (segment (start 214.5 102) (end 216 103.5) (width 0.2) (layer "F.Cu") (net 9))
 (segment (start 203.5 95.45) (end 203.5 102) (width 0.2) (layer "F.Cu") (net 9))
 (via (at 189 120) (size 0.6) (drill 0.3) (layers "F.Cu" "B.Cu") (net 9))
 (via (at 189.5 116) (size 0.6) (drill 0.3) (layers "F.Cu" "B.Cu") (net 9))
 (via (at 203.5 113) (size 0.6) (drill 0.3) (layers "F.Cu" "B.Cu") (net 9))
 (via (at 189 118.5) (size 0.6) (drill 0.3) (layers "F.Cu" "B.Cu") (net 9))
 (segment (start 203.5 113) (end 203.5 117) (width 0.2) (layer "B.Cu") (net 9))
 (segment (start 189 118.5) (end 189 116.5) (width 0.2) (layer "B.Cu") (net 9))
 (segment (start 203.5 117) (end 200.9 119.6) (width 0.2) (layer "B.Cu") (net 9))
 (segment (start 200.9 119.6) (end 189.4 119.6) (width 0.2) (layer "B.Cu") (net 9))
 (segment (start 189 116.5) (end 189.5 116) (width 0.2) (layer "B.Cu") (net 9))
 (segment (start 189.4 119.6) (end 189 120) (width 0.2) (layer "B.Cu") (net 9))
 (segment (start 206 73.5) (end 211.5 73.5) (width 0.2) (layer "F.Cu") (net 10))
 (segment (start 213 97.65) (end 214.35 99) (width 0.2) (layer "F.Cu") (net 10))
 (segment (start 214.35 99) (end 219.5 99) (width 0.2) (layer "F.Cu") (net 10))
 (segment (start 207.4 77.4) (end 206 76) (width 0.2) (layer "F.Cu") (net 10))
 (segment (start 217.5 108.5) (end 205.4 120.6) (width 0.2) (layer "F.Cu") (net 10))
 (segment (start 213 96.7) (end 213 99.934314) (width 0.2) (layer "F.Cu") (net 10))
 (segment (start 212.95 74.95) (end 212.95 77.4) (width 0.2) (layer "F.Cu") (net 10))
 (segment (start 215 77.5) (end 214.9 77.4) (width 0.2) (layer "F.Cu") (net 10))
 (segment (start 211.5 73.5) (end 212.95 74.95) (width 0.2) (layer "F.Cu") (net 10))
 (segment (start 213 96.7) (end 213 97.65) (width 0.2) (layer "F.Cu") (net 10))
 (segment (start 205.4 120.6) (end 188.6 120.6) (width 0.2) (layer "F.Cu") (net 10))
 (segment (start 214.9 77.4) (end 212.95 77.4) (width 0.2) (layer "F.Cu") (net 10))
 (segment (start 183.75 115.75) (end 183.75 114.32) (width 0.2) (layer "F.Cu") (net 10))
 (segment (start 208.85 77.4) (end 207.4 77.4) (width 0.2) (layer "F.Cu") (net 10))
 (segment (start 217.5 104.434314) (end 217.5 108.5) (width 0.2) (layer "F.Cu") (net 10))
 (segment (start 219.5 84.4074) (end 215.5 80.4074) (width 0.2) (layer "F.Cu") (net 10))
 (segment (start 215.5 80.4074) (end 215.5 77.5) (width 0.2) (layer "F.Cu") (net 10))
 (segment (start 219.5 99) (end 219.5 84.4074) (width 0.2) (layer "F.Cu") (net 10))
 (segment (start 206 76) (end 206 73.5) (width 0.2) (layer "F.Cu") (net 10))
 (segment (start 213 99.934314) (end 217.5 104.434314) (width 0.2) (layer "F.Cu") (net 10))
 (segment (start 215.5 77.5) (end 215 77.5) (width 0.2) (layer "F.Cu") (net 10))
 (segment (start 188.6 120.6) (end 183.75 115.75) (width 0.2) (layer "F.Cu") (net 10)))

